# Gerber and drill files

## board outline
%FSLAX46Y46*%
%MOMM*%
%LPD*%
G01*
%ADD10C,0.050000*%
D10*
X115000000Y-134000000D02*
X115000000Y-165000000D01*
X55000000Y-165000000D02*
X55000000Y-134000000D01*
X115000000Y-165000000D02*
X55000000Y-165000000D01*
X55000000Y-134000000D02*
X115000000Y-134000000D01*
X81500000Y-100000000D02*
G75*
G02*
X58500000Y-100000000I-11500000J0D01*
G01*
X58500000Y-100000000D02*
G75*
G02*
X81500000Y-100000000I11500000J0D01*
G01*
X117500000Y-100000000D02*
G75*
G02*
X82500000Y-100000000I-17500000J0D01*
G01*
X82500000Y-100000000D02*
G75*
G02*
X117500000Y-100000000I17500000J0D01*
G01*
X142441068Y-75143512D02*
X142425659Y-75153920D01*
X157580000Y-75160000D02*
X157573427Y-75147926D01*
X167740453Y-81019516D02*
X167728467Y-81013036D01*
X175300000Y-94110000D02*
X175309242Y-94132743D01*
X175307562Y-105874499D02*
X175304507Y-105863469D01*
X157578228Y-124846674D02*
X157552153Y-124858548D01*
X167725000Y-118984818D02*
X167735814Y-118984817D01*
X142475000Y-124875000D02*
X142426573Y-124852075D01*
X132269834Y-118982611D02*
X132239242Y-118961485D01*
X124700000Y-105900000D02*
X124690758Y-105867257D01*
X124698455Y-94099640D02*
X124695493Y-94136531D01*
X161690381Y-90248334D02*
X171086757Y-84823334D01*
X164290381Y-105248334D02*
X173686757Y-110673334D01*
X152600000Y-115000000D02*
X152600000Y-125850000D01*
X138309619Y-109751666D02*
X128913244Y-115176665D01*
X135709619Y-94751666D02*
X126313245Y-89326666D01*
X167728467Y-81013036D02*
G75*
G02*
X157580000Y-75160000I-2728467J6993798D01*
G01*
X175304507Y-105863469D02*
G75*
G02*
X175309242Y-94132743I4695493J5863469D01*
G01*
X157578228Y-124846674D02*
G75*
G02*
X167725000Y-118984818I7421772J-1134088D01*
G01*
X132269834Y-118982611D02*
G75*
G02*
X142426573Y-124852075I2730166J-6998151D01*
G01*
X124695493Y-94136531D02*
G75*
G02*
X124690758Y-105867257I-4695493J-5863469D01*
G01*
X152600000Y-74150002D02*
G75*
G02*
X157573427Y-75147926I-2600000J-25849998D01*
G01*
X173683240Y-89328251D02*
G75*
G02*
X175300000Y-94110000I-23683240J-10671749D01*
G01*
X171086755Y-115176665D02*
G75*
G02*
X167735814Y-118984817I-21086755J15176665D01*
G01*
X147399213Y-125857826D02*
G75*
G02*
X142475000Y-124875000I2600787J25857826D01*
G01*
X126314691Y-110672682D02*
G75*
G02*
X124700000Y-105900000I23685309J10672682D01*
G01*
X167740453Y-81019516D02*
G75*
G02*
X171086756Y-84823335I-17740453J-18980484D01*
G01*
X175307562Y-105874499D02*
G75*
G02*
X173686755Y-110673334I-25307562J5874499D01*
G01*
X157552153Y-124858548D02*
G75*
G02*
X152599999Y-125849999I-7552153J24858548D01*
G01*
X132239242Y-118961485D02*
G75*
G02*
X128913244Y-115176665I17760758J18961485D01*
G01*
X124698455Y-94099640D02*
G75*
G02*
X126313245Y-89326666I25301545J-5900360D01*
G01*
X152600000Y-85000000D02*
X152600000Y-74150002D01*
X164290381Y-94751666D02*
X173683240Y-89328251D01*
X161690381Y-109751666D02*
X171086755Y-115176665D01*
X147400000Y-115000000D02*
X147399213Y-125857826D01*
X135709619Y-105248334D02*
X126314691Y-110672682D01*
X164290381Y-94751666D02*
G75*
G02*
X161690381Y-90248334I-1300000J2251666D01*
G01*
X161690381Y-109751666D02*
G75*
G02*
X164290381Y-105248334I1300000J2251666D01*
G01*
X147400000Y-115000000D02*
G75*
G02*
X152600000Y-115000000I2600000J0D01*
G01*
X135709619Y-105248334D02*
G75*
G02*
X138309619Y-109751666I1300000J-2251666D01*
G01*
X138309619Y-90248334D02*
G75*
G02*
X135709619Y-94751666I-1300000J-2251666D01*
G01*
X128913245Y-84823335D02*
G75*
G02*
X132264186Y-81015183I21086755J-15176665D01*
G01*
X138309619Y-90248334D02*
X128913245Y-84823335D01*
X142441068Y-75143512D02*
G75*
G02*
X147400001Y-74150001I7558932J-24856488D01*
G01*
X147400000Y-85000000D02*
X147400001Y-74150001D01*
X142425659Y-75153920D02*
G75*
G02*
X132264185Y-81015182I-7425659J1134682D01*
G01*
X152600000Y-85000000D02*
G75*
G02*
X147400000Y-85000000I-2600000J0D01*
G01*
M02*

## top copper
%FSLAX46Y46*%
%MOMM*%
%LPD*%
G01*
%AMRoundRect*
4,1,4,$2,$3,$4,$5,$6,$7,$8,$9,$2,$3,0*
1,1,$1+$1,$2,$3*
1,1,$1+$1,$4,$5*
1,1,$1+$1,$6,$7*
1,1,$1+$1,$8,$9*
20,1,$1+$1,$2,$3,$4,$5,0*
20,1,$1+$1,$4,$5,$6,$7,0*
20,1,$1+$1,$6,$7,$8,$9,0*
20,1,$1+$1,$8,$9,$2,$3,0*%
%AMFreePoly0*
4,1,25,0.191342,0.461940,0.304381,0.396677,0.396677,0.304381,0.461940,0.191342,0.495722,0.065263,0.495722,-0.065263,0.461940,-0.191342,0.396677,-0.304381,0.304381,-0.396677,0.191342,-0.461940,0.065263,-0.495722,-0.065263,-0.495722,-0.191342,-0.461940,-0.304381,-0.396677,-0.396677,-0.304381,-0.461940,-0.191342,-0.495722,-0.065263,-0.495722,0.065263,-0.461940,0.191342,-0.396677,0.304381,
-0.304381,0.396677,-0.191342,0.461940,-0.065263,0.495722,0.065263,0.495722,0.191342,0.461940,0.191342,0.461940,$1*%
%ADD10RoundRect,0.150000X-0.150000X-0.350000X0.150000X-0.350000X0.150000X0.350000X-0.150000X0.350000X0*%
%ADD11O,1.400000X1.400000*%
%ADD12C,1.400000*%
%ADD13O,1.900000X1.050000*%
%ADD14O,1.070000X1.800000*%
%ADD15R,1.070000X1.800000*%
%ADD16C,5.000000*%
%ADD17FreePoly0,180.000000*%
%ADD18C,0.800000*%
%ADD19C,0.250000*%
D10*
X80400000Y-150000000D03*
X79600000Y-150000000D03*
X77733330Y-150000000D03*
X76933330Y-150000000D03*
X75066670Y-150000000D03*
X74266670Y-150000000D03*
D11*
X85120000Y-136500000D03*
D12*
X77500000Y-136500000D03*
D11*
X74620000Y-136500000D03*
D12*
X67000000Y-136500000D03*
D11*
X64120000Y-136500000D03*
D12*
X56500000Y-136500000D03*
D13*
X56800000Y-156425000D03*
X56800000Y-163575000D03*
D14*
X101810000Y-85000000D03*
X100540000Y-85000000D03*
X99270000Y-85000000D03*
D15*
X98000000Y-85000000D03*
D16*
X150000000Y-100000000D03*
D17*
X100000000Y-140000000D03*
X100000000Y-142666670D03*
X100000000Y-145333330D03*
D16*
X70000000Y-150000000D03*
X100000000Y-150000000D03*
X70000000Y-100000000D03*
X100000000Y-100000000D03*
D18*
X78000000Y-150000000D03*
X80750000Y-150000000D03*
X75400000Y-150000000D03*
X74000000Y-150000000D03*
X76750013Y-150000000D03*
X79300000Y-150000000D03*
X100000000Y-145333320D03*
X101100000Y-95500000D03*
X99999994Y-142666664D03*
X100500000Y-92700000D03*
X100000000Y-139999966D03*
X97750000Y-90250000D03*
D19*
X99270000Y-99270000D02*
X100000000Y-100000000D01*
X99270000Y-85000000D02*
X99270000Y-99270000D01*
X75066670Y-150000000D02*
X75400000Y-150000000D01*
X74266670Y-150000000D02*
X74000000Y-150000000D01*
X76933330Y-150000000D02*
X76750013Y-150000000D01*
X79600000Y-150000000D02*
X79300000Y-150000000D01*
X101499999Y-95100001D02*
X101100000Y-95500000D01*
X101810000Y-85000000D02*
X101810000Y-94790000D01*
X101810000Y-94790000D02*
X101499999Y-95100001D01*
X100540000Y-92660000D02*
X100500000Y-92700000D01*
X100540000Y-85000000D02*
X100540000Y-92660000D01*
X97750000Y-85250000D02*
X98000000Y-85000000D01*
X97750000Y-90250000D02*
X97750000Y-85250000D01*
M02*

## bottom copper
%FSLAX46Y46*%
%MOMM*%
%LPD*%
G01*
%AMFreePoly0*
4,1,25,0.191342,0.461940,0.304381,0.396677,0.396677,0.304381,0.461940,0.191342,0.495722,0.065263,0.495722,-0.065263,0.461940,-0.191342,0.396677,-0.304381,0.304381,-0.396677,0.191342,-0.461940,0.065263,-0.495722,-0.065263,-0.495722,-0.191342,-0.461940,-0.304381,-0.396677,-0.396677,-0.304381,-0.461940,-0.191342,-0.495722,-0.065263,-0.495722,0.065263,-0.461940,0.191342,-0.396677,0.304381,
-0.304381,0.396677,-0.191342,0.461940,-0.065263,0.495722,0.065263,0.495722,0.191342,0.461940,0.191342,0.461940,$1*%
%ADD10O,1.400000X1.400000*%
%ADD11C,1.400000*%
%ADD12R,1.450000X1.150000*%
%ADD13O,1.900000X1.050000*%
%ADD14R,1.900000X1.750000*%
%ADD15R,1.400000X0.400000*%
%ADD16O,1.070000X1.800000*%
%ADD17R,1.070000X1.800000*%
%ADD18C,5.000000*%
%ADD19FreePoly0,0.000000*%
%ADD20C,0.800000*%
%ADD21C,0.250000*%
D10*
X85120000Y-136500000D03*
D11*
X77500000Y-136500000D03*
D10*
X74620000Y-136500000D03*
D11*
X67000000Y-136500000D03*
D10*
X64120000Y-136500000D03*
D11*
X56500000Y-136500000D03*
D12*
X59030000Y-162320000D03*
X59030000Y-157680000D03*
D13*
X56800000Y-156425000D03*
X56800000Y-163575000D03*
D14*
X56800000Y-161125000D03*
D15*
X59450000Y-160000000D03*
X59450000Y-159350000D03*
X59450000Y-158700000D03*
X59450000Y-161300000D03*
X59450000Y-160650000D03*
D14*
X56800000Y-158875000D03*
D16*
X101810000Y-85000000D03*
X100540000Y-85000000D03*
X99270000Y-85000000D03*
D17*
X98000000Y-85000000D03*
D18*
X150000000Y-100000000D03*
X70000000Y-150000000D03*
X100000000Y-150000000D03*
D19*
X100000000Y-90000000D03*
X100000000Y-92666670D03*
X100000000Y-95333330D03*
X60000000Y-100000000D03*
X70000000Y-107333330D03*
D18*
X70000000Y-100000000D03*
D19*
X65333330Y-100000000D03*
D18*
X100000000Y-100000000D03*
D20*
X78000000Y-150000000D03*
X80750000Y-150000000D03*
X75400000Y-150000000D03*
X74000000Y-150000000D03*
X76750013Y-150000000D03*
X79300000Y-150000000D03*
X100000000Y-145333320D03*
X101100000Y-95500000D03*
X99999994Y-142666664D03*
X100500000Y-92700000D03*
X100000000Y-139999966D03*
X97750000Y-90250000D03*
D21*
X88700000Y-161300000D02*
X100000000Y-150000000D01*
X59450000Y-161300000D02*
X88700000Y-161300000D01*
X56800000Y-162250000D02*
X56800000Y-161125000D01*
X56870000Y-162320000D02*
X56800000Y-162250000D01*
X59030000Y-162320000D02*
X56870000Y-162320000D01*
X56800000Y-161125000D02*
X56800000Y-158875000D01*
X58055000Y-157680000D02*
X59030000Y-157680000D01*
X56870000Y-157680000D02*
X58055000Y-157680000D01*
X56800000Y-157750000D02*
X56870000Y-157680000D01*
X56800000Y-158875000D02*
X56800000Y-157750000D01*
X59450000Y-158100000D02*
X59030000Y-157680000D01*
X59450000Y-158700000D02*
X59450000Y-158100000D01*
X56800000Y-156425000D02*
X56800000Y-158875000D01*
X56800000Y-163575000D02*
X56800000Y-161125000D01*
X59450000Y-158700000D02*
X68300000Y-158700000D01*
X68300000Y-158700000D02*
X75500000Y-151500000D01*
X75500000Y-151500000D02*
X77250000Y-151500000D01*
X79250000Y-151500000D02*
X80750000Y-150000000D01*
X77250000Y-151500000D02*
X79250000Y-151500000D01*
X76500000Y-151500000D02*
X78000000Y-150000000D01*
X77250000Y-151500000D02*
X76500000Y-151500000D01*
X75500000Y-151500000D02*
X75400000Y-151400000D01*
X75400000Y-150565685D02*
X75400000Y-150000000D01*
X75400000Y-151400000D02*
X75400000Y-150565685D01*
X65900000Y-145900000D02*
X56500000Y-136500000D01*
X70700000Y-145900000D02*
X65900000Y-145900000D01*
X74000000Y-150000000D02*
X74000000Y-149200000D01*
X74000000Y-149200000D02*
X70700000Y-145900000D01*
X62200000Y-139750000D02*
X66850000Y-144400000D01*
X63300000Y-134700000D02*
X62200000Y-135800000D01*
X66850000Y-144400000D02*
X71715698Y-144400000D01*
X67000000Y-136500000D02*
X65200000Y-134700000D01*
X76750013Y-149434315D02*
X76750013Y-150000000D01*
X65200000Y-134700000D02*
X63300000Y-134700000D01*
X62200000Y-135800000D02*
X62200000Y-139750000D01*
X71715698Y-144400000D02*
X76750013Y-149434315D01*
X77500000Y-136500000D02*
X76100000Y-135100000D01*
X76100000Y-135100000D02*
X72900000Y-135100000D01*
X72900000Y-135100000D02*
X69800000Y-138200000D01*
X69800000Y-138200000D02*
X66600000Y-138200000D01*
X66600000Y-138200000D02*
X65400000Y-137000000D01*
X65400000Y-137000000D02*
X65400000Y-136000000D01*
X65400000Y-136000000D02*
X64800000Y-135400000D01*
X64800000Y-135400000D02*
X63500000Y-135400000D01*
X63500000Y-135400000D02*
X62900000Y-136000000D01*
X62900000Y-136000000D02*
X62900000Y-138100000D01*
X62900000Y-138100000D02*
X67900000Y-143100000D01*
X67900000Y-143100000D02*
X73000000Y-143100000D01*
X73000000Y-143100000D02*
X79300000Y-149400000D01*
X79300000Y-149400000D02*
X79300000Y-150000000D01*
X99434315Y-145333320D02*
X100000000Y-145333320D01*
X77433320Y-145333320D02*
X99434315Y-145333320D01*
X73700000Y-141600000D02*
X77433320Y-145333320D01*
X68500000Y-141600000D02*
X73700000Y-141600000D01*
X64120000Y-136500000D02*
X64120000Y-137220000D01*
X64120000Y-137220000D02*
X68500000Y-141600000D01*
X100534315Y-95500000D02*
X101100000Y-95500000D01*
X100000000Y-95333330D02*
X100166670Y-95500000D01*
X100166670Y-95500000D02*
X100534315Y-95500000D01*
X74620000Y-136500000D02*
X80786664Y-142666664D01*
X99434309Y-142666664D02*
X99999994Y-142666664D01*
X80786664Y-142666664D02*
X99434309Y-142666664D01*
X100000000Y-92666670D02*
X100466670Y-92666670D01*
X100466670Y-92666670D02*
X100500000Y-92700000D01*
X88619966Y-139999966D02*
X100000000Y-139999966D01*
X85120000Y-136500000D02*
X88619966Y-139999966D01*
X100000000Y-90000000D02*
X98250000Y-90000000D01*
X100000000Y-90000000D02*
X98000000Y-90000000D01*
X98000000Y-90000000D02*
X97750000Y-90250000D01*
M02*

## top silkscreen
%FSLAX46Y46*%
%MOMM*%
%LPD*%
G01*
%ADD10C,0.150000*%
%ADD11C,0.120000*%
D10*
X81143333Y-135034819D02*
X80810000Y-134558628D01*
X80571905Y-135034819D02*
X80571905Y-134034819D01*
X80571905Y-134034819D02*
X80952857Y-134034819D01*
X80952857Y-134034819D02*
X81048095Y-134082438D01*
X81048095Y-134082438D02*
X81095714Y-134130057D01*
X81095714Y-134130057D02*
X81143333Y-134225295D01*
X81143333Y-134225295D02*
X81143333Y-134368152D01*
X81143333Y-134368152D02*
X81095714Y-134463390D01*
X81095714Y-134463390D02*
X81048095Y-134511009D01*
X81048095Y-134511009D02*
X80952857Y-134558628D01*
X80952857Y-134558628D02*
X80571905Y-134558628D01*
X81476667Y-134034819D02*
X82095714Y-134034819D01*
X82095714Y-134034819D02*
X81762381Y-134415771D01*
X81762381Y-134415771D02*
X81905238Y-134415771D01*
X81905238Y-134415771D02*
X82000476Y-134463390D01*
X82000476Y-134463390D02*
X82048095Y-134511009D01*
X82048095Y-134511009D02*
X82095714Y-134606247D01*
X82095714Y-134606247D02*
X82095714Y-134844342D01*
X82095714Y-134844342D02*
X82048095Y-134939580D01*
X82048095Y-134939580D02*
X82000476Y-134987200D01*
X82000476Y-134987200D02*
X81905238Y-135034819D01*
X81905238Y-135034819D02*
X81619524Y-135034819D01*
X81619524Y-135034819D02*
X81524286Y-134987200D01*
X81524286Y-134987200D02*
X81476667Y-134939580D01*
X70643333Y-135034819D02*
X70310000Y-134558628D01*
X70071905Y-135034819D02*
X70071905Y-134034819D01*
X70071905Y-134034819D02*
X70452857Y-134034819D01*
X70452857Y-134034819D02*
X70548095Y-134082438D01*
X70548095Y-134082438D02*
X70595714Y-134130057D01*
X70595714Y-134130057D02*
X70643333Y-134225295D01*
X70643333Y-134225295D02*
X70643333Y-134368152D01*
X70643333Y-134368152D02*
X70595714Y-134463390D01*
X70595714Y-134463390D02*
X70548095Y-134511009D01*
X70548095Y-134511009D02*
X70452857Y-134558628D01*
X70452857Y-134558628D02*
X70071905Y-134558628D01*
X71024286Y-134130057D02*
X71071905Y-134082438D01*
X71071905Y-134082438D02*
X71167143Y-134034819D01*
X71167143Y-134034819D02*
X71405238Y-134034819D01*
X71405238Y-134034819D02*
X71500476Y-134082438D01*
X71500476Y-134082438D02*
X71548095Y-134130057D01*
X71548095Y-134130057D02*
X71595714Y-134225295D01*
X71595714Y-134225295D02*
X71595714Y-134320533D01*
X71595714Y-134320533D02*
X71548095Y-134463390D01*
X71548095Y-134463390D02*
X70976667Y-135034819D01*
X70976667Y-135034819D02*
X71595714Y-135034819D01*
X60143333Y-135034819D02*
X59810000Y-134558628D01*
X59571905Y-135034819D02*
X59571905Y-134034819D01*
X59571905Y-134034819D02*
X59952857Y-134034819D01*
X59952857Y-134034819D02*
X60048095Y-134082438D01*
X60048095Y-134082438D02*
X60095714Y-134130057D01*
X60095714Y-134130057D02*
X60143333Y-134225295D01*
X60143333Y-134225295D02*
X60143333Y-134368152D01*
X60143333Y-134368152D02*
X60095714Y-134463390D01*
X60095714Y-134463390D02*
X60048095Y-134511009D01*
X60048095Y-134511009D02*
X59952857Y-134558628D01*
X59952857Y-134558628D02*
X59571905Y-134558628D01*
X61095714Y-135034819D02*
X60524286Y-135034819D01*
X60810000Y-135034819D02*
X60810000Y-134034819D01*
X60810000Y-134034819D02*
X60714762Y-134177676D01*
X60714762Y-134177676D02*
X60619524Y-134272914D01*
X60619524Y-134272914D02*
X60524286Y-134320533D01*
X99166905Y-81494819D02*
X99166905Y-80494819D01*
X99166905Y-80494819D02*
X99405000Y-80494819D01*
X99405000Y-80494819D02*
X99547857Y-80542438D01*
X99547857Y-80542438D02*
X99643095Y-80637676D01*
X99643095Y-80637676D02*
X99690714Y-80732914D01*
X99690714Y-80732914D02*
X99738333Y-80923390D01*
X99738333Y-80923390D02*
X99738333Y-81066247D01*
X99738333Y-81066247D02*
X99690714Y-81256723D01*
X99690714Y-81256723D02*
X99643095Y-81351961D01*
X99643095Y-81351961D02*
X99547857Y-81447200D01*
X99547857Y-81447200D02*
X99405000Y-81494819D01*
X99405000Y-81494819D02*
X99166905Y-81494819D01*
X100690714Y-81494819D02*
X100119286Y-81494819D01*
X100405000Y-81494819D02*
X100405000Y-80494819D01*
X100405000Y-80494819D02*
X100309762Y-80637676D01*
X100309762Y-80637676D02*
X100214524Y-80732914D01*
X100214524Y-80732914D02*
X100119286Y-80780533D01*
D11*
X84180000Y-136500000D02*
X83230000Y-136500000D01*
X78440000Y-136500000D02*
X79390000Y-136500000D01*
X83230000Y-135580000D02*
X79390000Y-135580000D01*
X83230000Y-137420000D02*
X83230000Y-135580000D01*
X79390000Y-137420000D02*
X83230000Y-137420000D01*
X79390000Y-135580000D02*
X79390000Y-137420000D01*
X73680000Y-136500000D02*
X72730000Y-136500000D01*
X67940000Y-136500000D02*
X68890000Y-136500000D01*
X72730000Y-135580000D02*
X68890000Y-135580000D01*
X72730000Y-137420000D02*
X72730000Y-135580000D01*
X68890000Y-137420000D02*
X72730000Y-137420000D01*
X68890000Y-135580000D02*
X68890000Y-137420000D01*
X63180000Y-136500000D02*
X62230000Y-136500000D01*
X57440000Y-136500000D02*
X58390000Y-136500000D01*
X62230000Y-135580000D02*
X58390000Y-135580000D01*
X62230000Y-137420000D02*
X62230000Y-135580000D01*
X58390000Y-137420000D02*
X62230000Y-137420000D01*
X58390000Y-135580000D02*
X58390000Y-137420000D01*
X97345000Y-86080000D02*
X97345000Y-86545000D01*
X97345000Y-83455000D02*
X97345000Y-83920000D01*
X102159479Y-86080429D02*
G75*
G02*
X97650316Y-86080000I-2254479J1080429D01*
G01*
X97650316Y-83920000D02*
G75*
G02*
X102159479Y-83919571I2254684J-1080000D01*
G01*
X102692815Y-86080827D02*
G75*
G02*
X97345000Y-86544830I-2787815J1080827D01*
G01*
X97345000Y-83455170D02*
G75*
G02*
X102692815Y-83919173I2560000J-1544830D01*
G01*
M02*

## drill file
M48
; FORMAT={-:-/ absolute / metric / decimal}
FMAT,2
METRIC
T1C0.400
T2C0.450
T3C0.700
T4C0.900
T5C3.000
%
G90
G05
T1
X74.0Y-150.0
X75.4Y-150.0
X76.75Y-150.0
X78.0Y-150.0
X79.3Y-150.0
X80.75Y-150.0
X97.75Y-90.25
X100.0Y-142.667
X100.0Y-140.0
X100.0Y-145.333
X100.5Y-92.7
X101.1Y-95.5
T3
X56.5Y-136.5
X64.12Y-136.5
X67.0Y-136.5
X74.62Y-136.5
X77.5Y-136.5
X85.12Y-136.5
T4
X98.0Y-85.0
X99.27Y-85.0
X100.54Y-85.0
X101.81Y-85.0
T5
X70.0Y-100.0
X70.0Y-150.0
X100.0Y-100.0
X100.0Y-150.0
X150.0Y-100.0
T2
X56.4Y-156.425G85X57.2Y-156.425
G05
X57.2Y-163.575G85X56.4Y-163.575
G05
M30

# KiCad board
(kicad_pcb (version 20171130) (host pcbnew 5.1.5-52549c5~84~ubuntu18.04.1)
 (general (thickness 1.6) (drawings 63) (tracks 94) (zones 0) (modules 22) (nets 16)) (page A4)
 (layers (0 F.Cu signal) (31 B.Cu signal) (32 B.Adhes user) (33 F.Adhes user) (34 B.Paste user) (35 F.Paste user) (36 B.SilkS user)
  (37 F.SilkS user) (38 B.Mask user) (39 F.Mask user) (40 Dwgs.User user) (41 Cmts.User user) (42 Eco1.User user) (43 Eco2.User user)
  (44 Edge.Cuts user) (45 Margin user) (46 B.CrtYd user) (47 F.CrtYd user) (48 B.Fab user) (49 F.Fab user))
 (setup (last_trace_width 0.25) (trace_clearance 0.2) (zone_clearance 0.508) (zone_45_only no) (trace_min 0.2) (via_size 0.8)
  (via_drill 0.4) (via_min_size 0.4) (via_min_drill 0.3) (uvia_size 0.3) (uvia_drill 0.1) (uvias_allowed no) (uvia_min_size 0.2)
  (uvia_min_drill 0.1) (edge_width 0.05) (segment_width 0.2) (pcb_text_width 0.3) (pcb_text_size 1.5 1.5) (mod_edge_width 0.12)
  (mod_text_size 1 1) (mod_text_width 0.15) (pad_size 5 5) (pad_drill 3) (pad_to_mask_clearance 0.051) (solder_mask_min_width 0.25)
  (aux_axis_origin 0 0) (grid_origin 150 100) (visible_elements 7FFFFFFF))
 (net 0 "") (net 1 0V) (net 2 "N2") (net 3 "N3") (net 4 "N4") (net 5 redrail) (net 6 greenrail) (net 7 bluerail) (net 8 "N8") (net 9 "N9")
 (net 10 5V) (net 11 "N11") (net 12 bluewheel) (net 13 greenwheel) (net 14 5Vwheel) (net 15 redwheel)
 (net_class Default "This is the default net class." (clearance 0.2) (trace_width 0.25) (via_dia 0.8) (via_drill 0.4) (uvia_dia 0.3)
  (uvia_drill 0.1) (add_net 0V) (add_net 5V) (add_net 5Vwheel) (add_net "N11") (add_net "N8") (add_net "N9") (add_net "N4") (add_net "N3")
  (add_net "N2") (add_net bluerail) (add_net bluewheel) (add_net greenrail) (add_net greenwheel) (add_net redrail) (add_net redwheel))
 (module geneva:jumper (layer F.Cu) (at 80 150)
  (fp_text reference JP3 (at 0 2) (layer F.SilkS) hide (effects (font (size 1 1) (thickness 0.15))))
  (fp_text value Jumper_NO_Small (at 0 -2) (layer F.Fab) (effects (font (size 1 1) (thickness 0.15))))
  (pad 2 smd roundrect (at 0.4 0) (size 0.6 1) (layers F.Cu F.Mask) (roundrect_rratio 0.25) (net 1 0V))
  (pad 1 smd roundrect (at -0.4 0) (size 0.6 1) (layers F.Cu F.Mask) (roundrect_rratio 0.25) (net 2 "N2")))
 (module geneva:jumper (layer F.Cu) (at 77.33333 150)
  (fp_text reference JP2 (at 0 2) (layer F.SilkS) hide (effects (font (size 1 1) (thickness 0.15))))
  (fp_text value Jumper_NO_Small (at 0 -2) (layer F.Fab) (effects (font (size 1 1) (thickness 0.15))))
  (pad 2 smd roundrect (at 0.4 0) (size 0.6 1) (layers F.Cu F.Mask) (roundrect_rratio 0.25) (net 1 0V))
  (pad 1 smd roundrect (at -0.4 0) (size 0.6 1) (layers F.Cu F.Mask) (roundrect_rratio 0.25) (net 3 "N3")))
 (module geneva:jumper (layer F.Cu) (at 74.66667 150)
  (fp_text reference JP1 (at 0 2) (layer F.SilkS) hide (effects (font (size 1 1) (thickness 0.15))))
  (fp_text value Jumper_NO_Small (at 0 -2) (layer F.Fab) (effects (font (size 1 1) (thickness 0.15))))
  (pad 2 smd roundrect (at 0.4 0) (size 0.6 1) (layers F.Cu F.Mask) (roundrect_rratio 0.25) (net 1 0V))
  (pad 1 smd roundrect (at -0.4 0) (size 0.6 1) (layers F.Cu F.Mask) (roundrect_rratio 0.25) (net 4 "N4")))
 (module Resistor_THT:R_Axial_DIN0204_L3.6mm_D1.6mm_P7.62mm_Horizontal (layer F.Cu) (at 77.5 136.5)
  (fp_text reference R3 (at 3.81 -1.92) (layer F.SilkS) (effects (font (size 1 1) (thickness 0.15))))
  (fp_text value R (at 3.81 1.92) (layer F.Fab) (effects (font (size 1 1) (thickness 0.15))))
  (fp_line (start 6.68 0) (end 5.73 0) (layer F.SilkS) (width 0.12))
  (fp_line (start 0.94 0) (end 1.89 0) (layer F.SilkS) (width 0.12))
  (fp_line (start 5.73 -0.92) (end 1.89 -0.92) (layer F.SilkS) (width 0.12))
  (fp_line (start 5.73 0.92) (end 5.73 -0.92) (layer F.SilkS) (width 0.12))
  (fp_line (start 1.89 0.92) (end 5.73 0.92) (layer F.SilkS) (width 0.12))
  (fp_line (start 1.89 -0.92) (end 1.89 0.92) (layer F.SilkS) (width 0.12))
  (pad 2 thru_hole oval (at 7.62 0) (size 1.4 1.4) (drill 0.7) (layers *.Cu *.Mask) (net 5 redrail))
  (pad 1 thru_hole circle (at 0 0) (size 1.4 1.4) (drill 0.7) (layers *.Cu *.Mask) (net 2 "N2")))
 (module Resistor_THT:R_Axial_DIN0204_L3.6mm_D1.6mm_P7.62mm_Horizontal (layer F.Cu) (at 67 136.5)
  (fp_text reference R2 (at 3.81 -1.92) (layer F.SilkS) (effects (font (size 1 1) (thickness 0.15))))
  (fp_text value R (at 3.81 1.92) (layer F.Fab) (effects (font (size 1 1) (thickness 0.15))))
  (fp_line (start 6.68 0) (end 5.73 0) (layer F.SilkS) (width 0.12))
  (fp_line (start 0.94 0) (end 1.89 0) (layer F.SilkS) (width 0.12))
  (fp_line (start 5.73 -0.92) (end 1.89 -0.92) (layer F.SilkS) (width 0.12))
  (fp_line (start 5.73 0.92) (end 5.73 -0.92) (layer F.SilkS) (width 0.12))
  (fp_line (start 1.89 0.92) (end 5.73 0.92) (layer F.SilkS) (width 0.12))
  (fp_line (start 1.89 -0.92) (end 1.89 0.92) (layer F.SilkS) (width 0.12))
  (pad 2 thru_hole oval (at 7.62 0) (size 1.4 1.4) (drill 0.7) (layers *.Cu *.Mask) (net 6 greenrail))
  (pad 1 thru_hole circle (at 0 0) (size 1.4 1.4) (drill 0.7) (layers *.Cu *.Mask) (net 3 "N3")))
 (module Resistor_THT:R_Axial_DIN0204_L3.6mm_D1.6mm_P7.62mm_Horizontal (layer F.Cu) (at 56.5 136.5)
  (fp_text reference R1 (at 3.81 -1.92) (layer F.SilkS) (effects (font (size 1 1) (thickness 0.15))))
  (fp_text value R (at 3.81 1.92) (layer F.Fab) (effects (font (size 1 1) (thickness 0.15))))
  (fp_line (start 6.68 0) (end 5.73 0) (layer F.SilkS) (width 0.12))
  (fp_line (start 0.94 0) (end 1.89 0) (layer F.SilkS) (width 0.12))
  (fp_line (start 5.73 -0.92) (end 1.89 -0.92) (layer F.SilkS) (width 0.12))
  (fp_line (start 5.73 0.92) (end 5.73 -0.92) (layer F.SilkS) (width 0.12))
  (fp_line (start 1.89 0.92) (end 5.73 0.92) (layer F.SilkS) (width 0.12))
  (fp_line (start 1.89 -0.92) (end 1.89 0.92) (layer F.SilkS) (width 0.12))
  (pad 2 thru_hole oval (at 7.62 0) (size 1.4 1.4) (drill 0.7) (layers *.Cu *.Mask) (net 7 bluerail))
  (pad 1 thru_hole circle (at 0 0) (size 1.4 1.4) (drill 0.7) (layers *.Cu *.Mask) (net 4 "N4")))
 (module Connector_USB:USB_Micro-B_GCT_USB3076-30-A (layer B.Cu) (at 58 160 90)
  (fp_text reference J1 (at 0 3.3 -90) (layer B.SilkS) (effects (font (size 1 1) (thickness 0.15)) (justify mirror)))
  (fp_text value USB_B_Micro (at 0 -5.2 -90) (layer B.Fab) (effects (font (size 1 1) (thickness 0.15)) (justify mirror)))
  (pad 6 smd rect (at -2.32 1.03 90) (size 1.15 1.45) (layers B.Cu B.Paste B.Mask) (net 1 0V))
  (pad 6 smd rect (at 2.32 1.03 90) (size 1.15 1.45) (layers B.Cu B.Paste B.Mask) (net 1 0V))
  (pad 6 thru_hole oval (at 3.575 -1.2 90) (size 1.05 1.9) (drill oval 0.45 1.25) (layers *.Cu *.Mask) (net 1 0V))
  (pad 6 thru_hole oval (at -3.575 -1.2 270) (size 1.05 1.9) (drill oval 0.45 1.25) (layers *.Cu *.Mask) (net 1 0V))
  (pad 6 smd rect (at -1.125 -1.2 90) (size 1.75 1.9) (layers B.Cu B.Paste B.Mask) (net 1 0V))
  (pad 3 smd rect (at 0 1.45 90) (size 0.4 1.4) (layers B.Cu B.Paste B.Mask) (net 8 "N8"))
  (pad 4 smd rect (at 0.65 1.45 90) (size 0.4 1.4) (layers B.Cu B.Paste B.Mask) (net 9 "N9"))
  (pad 5 smd rect (at 1.3 1.45 90) (size 0.4 1.4) (layers B.Cu B.Paste B.Mask) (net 1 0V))
  (pad 1 smd rect (at -1.3 1.45 90) (size 0.4 1.4) (layers B.Cu B.Paste B.Mask) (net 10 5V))
  (pad 2 smd rect (at -0.65 1.45 90) (size 0.4 1.4) (layers B.Cu B.Paste B.Mask) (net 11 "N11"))
  (pad 6 smd rect (at 1.125 -1.2 90) (size 1.75 1.9) (layers B.Cu B.Paste B.Mask) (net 1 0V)))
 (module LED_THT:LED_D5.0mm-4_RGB (layer F.Cu) (at 98 85)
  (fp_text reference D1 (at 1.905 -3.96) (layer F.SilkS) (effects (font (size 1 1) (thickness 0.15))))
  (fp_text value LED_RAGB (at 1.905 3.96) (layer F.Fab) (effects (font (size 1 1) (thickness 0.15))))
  (fp_line (start -0.655 1.08) (end -0.655 1.545) (layer F.SilkS) (width 0.12))
  (fp_line (start -0.655 -1.545) (end -0.655 -1.08) (layer F.SilkS) (width 0.12))
  (fp_arc (start 1.905 0) (end -0.349684 1.08) (angle -128.8) (layer F.SilkS) (width 0.12))
  (fp_arc (start 1.905 0) (end -0.349684 -1.08) (angle 128.8) (layer F.SilkS) (width 0.12))
  (fp_arc (start 1.905 0) (end -0.655 1.54483) (angle -127.7) (layer F.SilkS) (width 0.12))
  (fp_arc (start 1.905 0) (end -0.655 -1.54483) (angle 127.7) (layer F.SilkS) (width 0.12))
  (pad 4 thru_hole oval (at 3.81 0) (size 1.07 1.8) (drill 0.9) (layers *.Cu *.Mask) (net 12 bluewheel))
  (pad 3 thru_hole oval (at 2.54 0) (size 1.07 1.8) (drill 0.9) (layers *.Cu *.Mask) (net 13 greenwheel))
  (pad 2 thru_hole oval (at 1.27 0) (size 1.07 1.8) (drill 0.9) (layers *.Cu *.Mask) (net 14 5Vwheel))
  (pad 1 thru_hole rect (at 0 0) (size 1.07 1.8) (drill 0.9) (layers *.Cu *.Mask) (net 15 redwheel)))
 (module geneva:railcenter (layer F.Cu) (at 150 100)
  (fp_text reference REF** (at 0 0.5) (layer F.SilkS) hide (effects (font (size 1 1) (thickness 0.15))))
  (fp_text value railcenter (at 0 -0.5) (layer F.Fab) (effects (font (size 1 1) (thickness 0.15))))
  (pad 1 thru_hole circle (at 0 0) (size 5 5) (drill 3) (layers *.Cu *.Mask)))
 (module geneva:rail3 (layer F.Cu) (at 100 150 180)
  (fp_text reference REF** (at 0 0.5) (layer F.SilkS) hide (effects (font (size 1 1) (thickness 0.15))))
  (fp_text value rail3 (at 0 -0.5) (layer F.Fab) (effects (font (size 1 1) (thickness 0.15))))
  (pad 1 smd custom (at 0 10 180) (size 1 1) (layers F.Cu F.Mask) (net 5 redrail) (zone_connect 0)
   (options (clearance outline) (anchor circle)) (primitives)))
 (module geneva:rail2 (layer F.Cu) (at 100 150 180)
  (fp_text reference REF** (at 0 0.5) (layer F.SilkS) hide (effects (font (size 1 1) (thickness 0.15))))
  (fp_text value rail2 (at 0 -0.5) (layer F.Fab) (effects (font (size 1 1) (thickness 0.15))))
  (pad 1 smd custom (at 0 7.33333 180) (size 1 1) (layers F.Cu F.Mask) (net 6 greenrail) (zone_connect 0)
   (options (clearance outline) (anchor circle)) (primitives)))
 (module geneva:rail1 (layer F.Cu) (at 100 150 180)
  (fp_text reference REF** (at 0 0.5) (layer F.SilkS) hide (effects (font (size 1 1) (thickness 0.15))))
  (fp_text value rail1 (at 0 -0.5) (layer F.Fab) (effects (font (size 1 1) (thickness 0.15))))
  (pad 1 smd custom (at 0 4.66667 180) (size 1 1) (layers F.Cu F.Mask) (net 7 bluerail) (zone_connect 0)
   (options (clearance outline) (anchor circle)) (primitives)))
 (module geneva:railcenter (layer F.Cu) (at 70 150)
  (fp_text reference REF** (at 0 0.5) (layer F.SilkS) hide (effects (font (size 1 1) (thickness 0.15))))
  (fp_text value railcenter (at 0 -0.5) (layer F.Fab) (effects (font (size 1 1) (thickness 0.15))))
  (pad 1 thru_hole circle (at 0 0) (size 5 5) (drill 3) (layers *.Cu *.Mask)))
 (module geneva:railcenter (layer F.Cu) (at 100 150)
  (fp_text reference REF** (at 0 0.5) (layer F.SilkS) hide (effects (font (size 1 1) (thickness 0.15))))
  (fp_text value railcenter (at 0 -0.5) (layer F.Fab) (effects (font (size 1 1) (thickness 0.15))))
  (pad 1 thru_hole circle (at 0 0) (size 5 5) (drill 3) (layers *.Cu *.Mask) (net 10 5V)))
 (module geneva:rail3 (layer B.Cu) (at 100 100)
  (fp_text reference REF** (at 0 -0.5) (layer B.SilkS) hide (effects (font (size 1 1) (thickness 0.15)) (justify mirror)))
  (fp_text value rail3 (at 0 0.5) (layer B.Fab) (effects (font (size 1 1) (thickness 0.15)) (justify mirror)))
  (pad 1 smd custom (at 0 -10) (size 1 1) (layers B.Cu B.Mask) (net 15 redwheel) (zone_connect 0)
   (options (clearance outline) (anchor circle)) (primitives)))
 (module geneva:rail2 (layer B.Cu) (at 100 100)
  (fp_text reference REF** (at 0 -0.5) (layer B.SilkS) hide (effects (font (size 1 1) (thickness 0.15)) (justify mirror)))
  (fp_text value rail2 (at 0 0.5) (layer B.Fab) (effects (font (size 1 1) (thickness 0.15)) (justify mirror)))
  (pad 1 smd custom (at 0 -7.33333) (size 1 1) (layers B.Cu B.Mask) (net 13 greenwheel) (zone_connect 0)
   (options (clearance outline) (anchor circle)) (primitives)))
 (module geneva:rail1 (layer B.Cu) (at 100 100)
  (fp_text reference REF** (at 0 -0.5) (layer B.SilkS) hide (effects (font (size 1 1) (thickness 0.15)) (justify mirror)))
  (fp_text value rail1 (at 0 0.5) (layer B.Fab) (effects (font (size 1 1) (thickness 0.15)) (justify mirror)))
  (pad 1 smd custom (at 0 -4.66667) (size 1 1) (layers B.Cu B.Mask) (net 12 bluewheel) (zone_connect 0)
   (options (clearance outline) (anchor circle)) (primitives)))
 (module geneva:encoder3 (layer B.Cu) (at 70 100)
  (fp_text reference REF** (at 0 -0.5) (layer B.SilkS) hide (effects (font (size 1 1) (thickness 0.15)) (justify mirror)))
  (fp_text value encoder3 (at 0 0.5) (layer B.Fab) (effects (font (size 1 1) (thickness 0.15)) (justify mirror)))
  (pad 1 smd custom (at -10 0) (size 1 1) (layers B.Cu B.Mask) (zone_connect 0) (options (clearance outline) (anchor circle)) (primitives)))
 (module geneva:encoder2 (layer B.Cu) (at 70 100)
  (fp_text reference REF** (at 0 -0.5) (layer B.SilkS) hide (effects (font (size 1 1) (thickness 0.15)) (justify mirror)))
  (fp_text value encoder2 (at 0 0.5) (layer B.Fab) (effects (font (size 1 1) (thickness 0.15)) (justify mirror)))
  (pad 1 smd custom (at 0 7.33333) (size 1 1) (layers B.Cu B.Mask) (zone_connect 0) (options (clearance outline) (anchor circle))
   (primitives)))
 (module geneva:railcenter (layer F.Cu) (at 70 100)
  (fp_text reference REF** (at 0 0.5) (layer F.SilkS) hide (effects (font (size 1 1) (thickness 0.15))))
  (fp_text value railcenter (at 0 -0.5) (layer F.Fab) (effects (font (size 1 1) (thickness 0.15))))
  (pad 1 thru_hole circle (at 0 0) (size 5 5) (drill 3) (layers *.Cu *.Mask)))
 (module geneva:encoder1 (layer B.Cu) (at 70 100)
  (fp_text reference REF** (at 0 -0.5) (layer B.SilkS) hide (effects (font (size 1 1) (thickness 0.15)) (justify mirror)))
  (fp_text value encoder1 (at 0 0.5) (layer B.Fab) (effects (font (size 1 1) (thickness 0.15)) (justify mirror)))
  (pad 1 smd custom (at -4.66667 0) (size 1 1) (layers B.Cu B.Mask) (zone_connect 0) (options (clearance outline) (anchor circle))
   (primitives)))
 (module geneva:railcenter (layer F.Cu) (at 100 100)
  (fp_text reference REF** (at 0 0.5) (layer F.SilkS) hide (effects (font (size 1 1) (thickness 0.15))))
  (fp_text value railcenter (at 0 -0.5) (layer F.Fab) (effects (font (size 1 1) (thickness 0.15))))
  (pad 1 thru_hole circle (at 0 0) (size 5 5) (drill 3) (layers *.Cu *.Mask) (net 14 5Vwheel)))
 (gr_line (start 115 134) (end 115 165) (layer Edge.Cuts) (width 0.05))
 (gr_line (start 55 165) (end 55 134) (layer Edge.Cuts) (width 0.05))
 (gr_line (start 115 165) (end 55 165) (layer Edge.Cuts) (width 0.05))
 (gr_line (start 55 134) (end 115 134) (layer Edge.Cuts) (width 0.05))
 (gr_circle (center 70 100) (end 81.5 100) (layer Edge.Cuts) (width 0.05))
 (gr_circle (center 100 100) (end 100 82.5) (layer Edge.Cuts) (width 0.05))
 (gr_line (start 142.441068 75.143512) (end 142.425659 75.15392) (layer Edge.Cuts) (width 0.05))
 (gr_line (start 157.58 75.16) (end 157.573427 75.147926) (layer Edge.Cuts) (width 0.05))
 (gr_line (start 167.740453 81.019516) (end 167.728467 81.013036) (layer Edge.Cuts) (width 0.05))
 (gr_line (start 175.3 94.11) (end 175.309242 94.132743) (layer Edge.Cuts) (width 0.05))
 (gr_line (start 175.307562 105.874499) (end 175.304507 105.863469) (layer Edge.Cuts) (width 0.05))
 (gr_line (start 157.578228 124.846674) (end 157.552153 124.858548) (layer Edge.Cuts) (width 0.05))
 (gr_line (start 167.725 118.984818) (end 167.735814 118.984817) (layer Edge.Cuts) (width 0.05))
 (gr_line (start 142.475 124.875) (end 142.426573 124.852075) (layer Edge.Cuts) (width 0.05))
 (gr_line (start 132.269834 118.982611) (end 132.239242 118.961485) (layer Edge.Cuts) (width 0.05))
 (gr_line (start 124.7 105.9) (end 124.690758 105.867257) (layer Edge.Cuts) (width 0.05))
 (gr_line (start 124.698455 94.09964) (end 124.695493 94.136531) (layer Edge.Cuts) (width 0.05))
 (gr_line (start 161.690381 90.248334) (end 171.086757 84.823334) (layer Edge.Cuts) (width 0.05))
 (gr_line (start 164.290381 105.248334) (end 173.686757 110.673334) (layer Edge.Cuts) (width 0.05))
 (gr_line (start 152.6 115) (end 152.6 125.85) (layer Edge.Cuts) (width 0.05))
 (gr_line (start 138.309619 109.751666) (end 128.913244 115.176665) (layer Edge.Cuts) (width 0.05))
 (gr_line (start 135.709619 94.751666) (end 126.313245 89.326666) (layer Edge.Cuts) (width 0.05))
 (gr_arc (start 165 74.019238) (end 157.58 75.16) (angle -102.5717765) (layer Edge.Cuts) (width 0.05))
 (gr_arc (start 180 100) (end 175.309242 94.132743) (angle -102.670436) (layer Edge.Cuts) (width 0.05))
 (gr_arc (start 165 125.980762) (end 167.725 118.984818) (angle -102.5935713) (layer Edge.Cuts) (width 0.05))
 (gr_arc (start 135 125.980762) (end 142.426573 124.852075) (angle -102.670436) (layer Edge.Cuts) (width 0.05))
 (gr_arc (start 120 100) (end 124.690758 105.867257) (angle -102.670436) (layer Edge.Cuts) (width 0.05))
 (gr_arc (start 150 100) (end 157.573427 75.147926) (angle -11.20457929) (layer Edge.Cuts) (width 0.05))
 (gr_arc (start 150 100) (end 175.3 94.11) (angle -11.15110758) (layer Edge.Cuts) (width 0.05))
 (gr_arc (start 150 100) (end 167.735814 118.984817) (angle -11.20457929) (layer Edge.Cuts) (width 0.05))
 (gr_arc (start 150 100) (end 142.475 124.875) (angle -11.08771661) (layer Edge.Cuts) (width 0.05))
 (gr_arc (start 150 100) (end 124.7 105.9) (angle -11.12962862) (layer Edge.Cuts) (width 0.05))
 (gr_arc (start 150 100) (end 171.086756 84.823335) (angle -11.1905817) (layer Edge.Cuts) (width 0.05))
 (gr_arc (start 150 100) (end 173.686755 110.673334) (angle -11.18818472) (layer Edge.Cuts) (width 0.05))
 (gr_arc (start 150 100) (end 152.599999 125.849999) (angle -11.15554124) (layer Edge.Cuts) (width 0.05))
 (gr_arc (start 150 100) (end 128.913244 115.176665) (angle -11.12925613) (layer Edge.Cuts) (width 0.05))
 (gr_arc (start 150 100) (end 126.313245 89.326666) (angle -11.12962948) (layer Edge.Cuts) (width 0.05))
 (gr_line (start 152.6 85) (end 152.6 74.150002) (layer Edge.Cuts) (width 0.05))
 (gr_line (start 164.290381 94.751666) (end 173.68324 89.328251) (layer Edge.Cuts) (width 0.05))
 (gr_line (start 161.690381 109.751666) (end 171.086755 115.176665) (layer Edge.Cuts) (width 0.05))
 (gr_line (start 147.4 115) (end 147.399213 125.857826) (layer Edge.Cuts) (width 0.05))
 (gr_line (start 135.709619 105.248334) (end 126.314691 110.672682) (layer Edge.Cuts) (width 0.05))
 (gr_arc (start 162.990381 92.5) (end 161.690381 90.248334) (angle -180) (layer Edge.Cuts) (width 0.05))
 (gr_arc (start 162.990381 107.5) (end 164.290381 105.248334) (angle -180) (layer Edge.Cuts) (width 0.05))
 (gr_arc (start 150 115) (end 152.6 115) (angle -180) (layer Edge.Cuts) (width 0.05))
 (gr_arc (start 137.009619 107.5) (end 138.309619 109.751666) (angle -180) (layer Edge.Cuts) (width 0.05))
 (gr_arc (start 137.009619 92.5) (end 135.709619 94.751666) (angle -180) (layer Edge.Cuts) (width 0.05))
 (gr_arc (start 150 100) (end 132.264186 81.015183) (angle -11.20457929) (layer Edge.Cuts) (width 0.05))
 (gr_line (start 138.309619 90.248334) (end 128.913245 84.823335) (layer Edge.Cuts) (width 0.05))
 (gr_arc (start 150 100) (end 147.400001 74.150001) (angle -11.17116549) (layer Edge.Cuts) (width 0.05))
 (gr_line (start 147.4 85) (end 147.400001 74.150001) (layer Edge.Cuts) (width 0.05))
 (gr_arc (start 135 74.019238) (end 132.264185 81.015182) (angle -102.670436) (layer Edge.Cuts) (width 0.05))
 (gr_arc (start 150 85) (end 147.4 85) (angle -180) (layer Edge.Cuts) (width 0.05))
 (segment (start 88.7 161.3) (end 100 150) (width 0.25) (layer B.Cu) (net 10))
 (segment (start 59.45 161.3) (end 88.7 161.3) (width 0.25) (layer B.Cu) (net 10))
 (segment (start 99.27 99.27) (end 100 100) (width 0.25) (layer F.Cu) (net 14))
 (segment (start 99.27 85) (end 99.27 99.27) (width 0.25) (layer F.Cu) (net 14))
 (segment (start 56.8 162.25) (end 56.8 161.125) (width 0.25) (layer B.Cu) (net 1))
 (segment (start 56.87 162.32) (end 56.8 162.25) (width 0.25) (layer B.Cu) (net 1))
 (segment (start 59.03 162.32) (end 56.87 162.32) (width 0.25) (layer B.Cu) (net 1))
 (segment (start 56.8 161.125) (end 56.8 158.875) (width 0.25) (layer B.Cu) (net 1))
 (segment (start 58.055 157.68) (end 59.03 157.68) (width 0.25) (layer B.Cu) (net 1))
 (segment (start 56.87 157.68) (end 58.055 157.68) (width 0.25) (layer B.Cu) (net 1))
 (segment (start 56.8 157.75) (end 56.87 157.68) (width 0.25) (layer B.Cu) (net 1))
 (segment (start 56.8 158.875) (end 56.8 157.75) (width 0.25) (layer B.Cu) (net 1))
 (segment (start 59.45 158.1) (end 59.03 157.68) (width 0.25) (layer B.Cu) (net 1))
 (segment (start 59.45 158.7) (end 59.45 158.1) (width 0.25) (layer B.Cu) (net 1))
 (segment (start 56.8 156.425) (end 56.8 158.875) (width 0.25) (layer B.Cu) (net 1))
 (segment (start 56.8 163.575) (end 56.8 161.125) (width 0.25) (layer B.Cu) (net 1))
 (segment (start 59.45 158.7) (end 68.3 158.7) (width 0.25) (layer B.Cu) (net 1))
 (segment (start 68.3 158.7) (end 75.5 151.5) (width 0.25) (layer B.Cu) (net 1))
 (segment (start 75.5 151.5) (end 77.25 151.5) (width 0.25) (layer B.Cu) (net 1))
 (via (at 78 150) (size 0.8) (drill 0.4) (layers F.Cu B.Cu) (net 1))
 (via (at 80.75 150) (size 0.8) (drill 0.4) (layers F.Cu B.Cu) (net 1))
 (segment (start 79.25 151.5) (end 80.75 150) (width 0.25) (layer B.Cu) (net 1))
 (segment (start 77.25 151.5) (end 79.25 151.5) (width 0.25) (layer B.Cu) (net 1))
 (segment (start 76.5 151.5) (end 78 150) (width 0.25) (layer B.Cu) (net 1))
 (segment (start 77.25 151.5) (end 76.5 151.5) (width 0.25) (layer B.Cu) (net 1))
 (segment (start 75.06667 150) (end 75.4 150) (width 0.25) (layer F.Cu) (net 1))
 (via (at 75.4 150) (size 0.8) (drill 0.4) (layers F.Cu B.Cu) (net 1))
 (segment (start 75.5 151.5) (end 75.4 151.4) (width 0.25) (layer B.Cu) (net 1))
 (segment (start 75.4 150.565685) (end 75.4 150) (width 0.25) (layer B.Cu) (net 1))
 (segment (start 75.4 151.4) (end 75.4 150.565685) (width 0.25) (layer B.Cu) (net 1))
 (via (at 74 150) (size 0.8) (drill 0.4) (layers F.Cu B.Cu) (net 4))
 (segment (start 74.26667 150) (end 74 150) (width 0.25) (layer F.Cu) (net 4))
 (segment (start 65.9 145.9) (end 56.5 136.5) (width 0.25) (layer B.Cu) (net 4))
 (segment (start 70.7 145.9) (end 65.9 145.9) (width 0.25) (layer B.Cu) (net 4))
 (segment (start 74 150) (end 74 149.2) (width 0.25) (layer B.Cu) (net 4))
 (segment (start 74 149.2) (end 70.7 145.9) (width 0.25) (layer B.Cu) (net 4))
 (segment (start 62.2 139.75) (end 66.85 144.4) (width 0.25) (layer B.Cu) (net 3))
 (segment (start 63.3 134.7) (end 62.2 135.8) (width 0.25) (layer B.Cu) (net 3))
 (segment (start 66.85 144.4) (end 71.715698 144.4) (width 0.25) (layer B.Cu) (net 3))
 (segment (start 67 136.5) (end 65.2 134.7) (width 0.25) (layer B.Cu) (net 3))
 (segment (start 76.750013 149.434315) (end 76.750013 150) (width 0.25) (layer B.Cu) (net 3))
 (segment (start 65.2 134.7) (end 63.3 134.7) (width 0.25) (layer B.Cu) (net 3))
 (segment (start 76.93333 150) (end 76.750013 150) (width 0.25) (layer F.Cu) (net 3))
 (segment (start 62.2 135.8) (end 62.2 139.75) (width 0.25) (layer B.Cu) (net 3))
 (via (at 76.750013 150) (size 0.8) (drill 0.4) (layers F.Cu B.Cu) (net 3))
 (segment (start 71.715698 144.4) (end 76.750013 149.434315) (width 0.25) (layer B.Cu) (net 3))
 (segment (start 77.5 136.5) (end 76.1 135.1) (width 0.25) (layer B.Cu) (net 2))
 (segment (start 76.1 135.1) (end 72.9 135.1) (width 0.25) (layer B.Cu) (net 2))
 (segment (start 72.9 135.1) (end 69.8 138.2) (width 0.25) (layer B.Cu) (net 2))
 (segment (start 69.8 138.2) (end 66.6 138.2) (width 0.25) (layer B.Cu) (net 2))
 (segment (start 66.6 138.2) (end 65.4 137) (width 0.25) (layer B.Cu) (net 2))
 (segment (start 65.4 137) (end 65.4 136) (width 0.25) (layer B.Cu) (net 2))
 (segment (start 65.4 136) (end 64.8 135.4) (width 0.25) (layer B.Cu) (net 2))
 (segment (start 64.8 135.4) (end 63.5 135.4) (width 0.25) (layer B.Cu) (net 2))
 (segment (start 63.5 135.4) (end 62.9 136) (width 0.25) (layer B.Cu) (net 2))
 (segment (start 62.9 136) (end 62.9 138.1) (width 0.25) (layer B.Cu) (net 2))
 (segment (start 62.9 138.1) (end 67.9 143.1) (width 0.25) (layer B.Cu) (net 2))
 (segment (start 67.9 143.1) (end 73 143.1) (width 0.25) (layer B.Cu) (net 2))
 (via (at 79.3 150) (size 0.8) (drill 0.4) (layers F.Cu B.Cu) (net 2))
 (segment (start 73 143.1) (end 79.3 149.4) (width 0.25) (layer B.Cu) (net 2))
 (segment (start 79.3 149.4) (end 79.3 150) (width 0.25) (layer B.Cu) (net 2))
 (segment (start 79.6 150) (end 79.3 150) (width 0.25) (layer F.Cu) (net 2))
 (via (at 100 145.33332) (size 0.8) (drill 0.4) (layers F.Cu B.Cu) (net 7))
 (segment (start 99.434315 145.33332) (end 100 145.33332) (width 0.25) (layer B.Cu) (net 7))
 (segment (start 77.43332 145.33332) (end 99.434315 145.33332) (width 0.25) (layer B.Cu) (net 7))
 (segment (start 73.7 141.6) (end 77.43332 145.33332) (width 0.25) (layer B.Cu) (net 7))
 (segment (start 68.5 141.6) (end 73.7 141.6) (width 0.25) (layer B.Cu) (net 7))
 (segment (start 64.12 136.5) (end 64.12 137.22) (width 0.25) (layer B.Cu) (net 7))
 (segment (start 64.12 137.22) (end 68.5 141.6) (width 0.25) (layer B.Cu) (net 7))
 (segment (start 100.534315 95.5) (end 101.1 95.5) (width 0.25) (layer B.Cu) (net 12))
 (segment (start 100 95.33333) (end 100.16667 95.5) (width 0.25) (layer B.Cu) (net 12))
 (segment (start 100.16667 95.5) (end 100.534315 95.5) (width 0.25) (layer B.Cu) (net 12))
 (via (at 101.1 95.5) (size 0.8) (drill 0.4) (layers F.Cu B.Cu) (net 12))
 (segment (start 101.499999 95.100001) (end 101.1 95.5) (width 0.25) (layer F.Cu) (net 12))
 (segment (start 101.81 85) (end 101.81 94.79) (width 0.25) (layer F.Cu) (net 12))
 (segment (start 101.81 94.79) (end 101.499999 95.100001) (width 0.25) (layer F.Cu) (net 12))
 (via (at 99.999994 142.666664) (size 0.8) (drill 0.4) (layers F.Cu B.Cu) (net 6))
 (segment (start 74.62 136.5) (end 80.786664 142.666664) (width 0.25) (layer B.Cu) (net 6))
 (segment (start 99.434309 142.666664) (end 99.999994 142.666664) (width 0.25) (layer B.Cu) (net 6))
 (segment (start 80.786664 142.666664) (end 99.434309 142.666664) (width 0.25) (layer B.Cu) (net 6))
 (via (at 100.5 92.7) (size 0.8) (drill 0.4) (layers F.Cu B.Cu) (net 13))
 (segment (start 100 92.66667) (end 100.46667 92.66667) (width 0.25) (layer B.Cu) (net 13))
 (segment (start 100.46667 92.66667) (end 100.5 92.7) (width 0.25) (layer B.Cu) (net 13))
 (segment (start 100.54 92.66) (end 100.5 92.7) (width 0.25) (layer F.Cu) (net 13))
 (segment (start 100.54 85) (end 100.54 92.66) (width 0.25) (layer F.Cu) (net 13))
 (via (at 100 139.999966) (size 0.8) (drill 0.4) (layers F.Cu B.Cu) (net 5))
 (segment (start 88.619966 139.999966) (end 100 139.999966) (width 0.25) (layer B.Cu) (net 5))
 (segment (start 85.12 136.5) (end 88.619966 139.999966) (width 0.25) (layer B.Cu) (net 5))
 (segment (start 100 90) (end 98.25 90) (width 0.25) (layer B.Cu) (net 15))
 (via (at 97.75 90.25) (size 0.8) (drill 0.4) (layers F.Cu B.Cu) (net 15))
 (segment (start 100 90) (end 98 90) (width 0.25) (layer B.Cu) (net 15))
 (segment (start 98 90) (end 97.75 90.25) (width 0.25) (layer B.Cu) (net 15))
 (segment (start 97.75 85.25) (end 98 85) (width 0.25) (layer F.Cu) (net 15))
 (segment (start 97.75 90.25) (end 97.75 85.25) (width 0.25) (layer F.Cu) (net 15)))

